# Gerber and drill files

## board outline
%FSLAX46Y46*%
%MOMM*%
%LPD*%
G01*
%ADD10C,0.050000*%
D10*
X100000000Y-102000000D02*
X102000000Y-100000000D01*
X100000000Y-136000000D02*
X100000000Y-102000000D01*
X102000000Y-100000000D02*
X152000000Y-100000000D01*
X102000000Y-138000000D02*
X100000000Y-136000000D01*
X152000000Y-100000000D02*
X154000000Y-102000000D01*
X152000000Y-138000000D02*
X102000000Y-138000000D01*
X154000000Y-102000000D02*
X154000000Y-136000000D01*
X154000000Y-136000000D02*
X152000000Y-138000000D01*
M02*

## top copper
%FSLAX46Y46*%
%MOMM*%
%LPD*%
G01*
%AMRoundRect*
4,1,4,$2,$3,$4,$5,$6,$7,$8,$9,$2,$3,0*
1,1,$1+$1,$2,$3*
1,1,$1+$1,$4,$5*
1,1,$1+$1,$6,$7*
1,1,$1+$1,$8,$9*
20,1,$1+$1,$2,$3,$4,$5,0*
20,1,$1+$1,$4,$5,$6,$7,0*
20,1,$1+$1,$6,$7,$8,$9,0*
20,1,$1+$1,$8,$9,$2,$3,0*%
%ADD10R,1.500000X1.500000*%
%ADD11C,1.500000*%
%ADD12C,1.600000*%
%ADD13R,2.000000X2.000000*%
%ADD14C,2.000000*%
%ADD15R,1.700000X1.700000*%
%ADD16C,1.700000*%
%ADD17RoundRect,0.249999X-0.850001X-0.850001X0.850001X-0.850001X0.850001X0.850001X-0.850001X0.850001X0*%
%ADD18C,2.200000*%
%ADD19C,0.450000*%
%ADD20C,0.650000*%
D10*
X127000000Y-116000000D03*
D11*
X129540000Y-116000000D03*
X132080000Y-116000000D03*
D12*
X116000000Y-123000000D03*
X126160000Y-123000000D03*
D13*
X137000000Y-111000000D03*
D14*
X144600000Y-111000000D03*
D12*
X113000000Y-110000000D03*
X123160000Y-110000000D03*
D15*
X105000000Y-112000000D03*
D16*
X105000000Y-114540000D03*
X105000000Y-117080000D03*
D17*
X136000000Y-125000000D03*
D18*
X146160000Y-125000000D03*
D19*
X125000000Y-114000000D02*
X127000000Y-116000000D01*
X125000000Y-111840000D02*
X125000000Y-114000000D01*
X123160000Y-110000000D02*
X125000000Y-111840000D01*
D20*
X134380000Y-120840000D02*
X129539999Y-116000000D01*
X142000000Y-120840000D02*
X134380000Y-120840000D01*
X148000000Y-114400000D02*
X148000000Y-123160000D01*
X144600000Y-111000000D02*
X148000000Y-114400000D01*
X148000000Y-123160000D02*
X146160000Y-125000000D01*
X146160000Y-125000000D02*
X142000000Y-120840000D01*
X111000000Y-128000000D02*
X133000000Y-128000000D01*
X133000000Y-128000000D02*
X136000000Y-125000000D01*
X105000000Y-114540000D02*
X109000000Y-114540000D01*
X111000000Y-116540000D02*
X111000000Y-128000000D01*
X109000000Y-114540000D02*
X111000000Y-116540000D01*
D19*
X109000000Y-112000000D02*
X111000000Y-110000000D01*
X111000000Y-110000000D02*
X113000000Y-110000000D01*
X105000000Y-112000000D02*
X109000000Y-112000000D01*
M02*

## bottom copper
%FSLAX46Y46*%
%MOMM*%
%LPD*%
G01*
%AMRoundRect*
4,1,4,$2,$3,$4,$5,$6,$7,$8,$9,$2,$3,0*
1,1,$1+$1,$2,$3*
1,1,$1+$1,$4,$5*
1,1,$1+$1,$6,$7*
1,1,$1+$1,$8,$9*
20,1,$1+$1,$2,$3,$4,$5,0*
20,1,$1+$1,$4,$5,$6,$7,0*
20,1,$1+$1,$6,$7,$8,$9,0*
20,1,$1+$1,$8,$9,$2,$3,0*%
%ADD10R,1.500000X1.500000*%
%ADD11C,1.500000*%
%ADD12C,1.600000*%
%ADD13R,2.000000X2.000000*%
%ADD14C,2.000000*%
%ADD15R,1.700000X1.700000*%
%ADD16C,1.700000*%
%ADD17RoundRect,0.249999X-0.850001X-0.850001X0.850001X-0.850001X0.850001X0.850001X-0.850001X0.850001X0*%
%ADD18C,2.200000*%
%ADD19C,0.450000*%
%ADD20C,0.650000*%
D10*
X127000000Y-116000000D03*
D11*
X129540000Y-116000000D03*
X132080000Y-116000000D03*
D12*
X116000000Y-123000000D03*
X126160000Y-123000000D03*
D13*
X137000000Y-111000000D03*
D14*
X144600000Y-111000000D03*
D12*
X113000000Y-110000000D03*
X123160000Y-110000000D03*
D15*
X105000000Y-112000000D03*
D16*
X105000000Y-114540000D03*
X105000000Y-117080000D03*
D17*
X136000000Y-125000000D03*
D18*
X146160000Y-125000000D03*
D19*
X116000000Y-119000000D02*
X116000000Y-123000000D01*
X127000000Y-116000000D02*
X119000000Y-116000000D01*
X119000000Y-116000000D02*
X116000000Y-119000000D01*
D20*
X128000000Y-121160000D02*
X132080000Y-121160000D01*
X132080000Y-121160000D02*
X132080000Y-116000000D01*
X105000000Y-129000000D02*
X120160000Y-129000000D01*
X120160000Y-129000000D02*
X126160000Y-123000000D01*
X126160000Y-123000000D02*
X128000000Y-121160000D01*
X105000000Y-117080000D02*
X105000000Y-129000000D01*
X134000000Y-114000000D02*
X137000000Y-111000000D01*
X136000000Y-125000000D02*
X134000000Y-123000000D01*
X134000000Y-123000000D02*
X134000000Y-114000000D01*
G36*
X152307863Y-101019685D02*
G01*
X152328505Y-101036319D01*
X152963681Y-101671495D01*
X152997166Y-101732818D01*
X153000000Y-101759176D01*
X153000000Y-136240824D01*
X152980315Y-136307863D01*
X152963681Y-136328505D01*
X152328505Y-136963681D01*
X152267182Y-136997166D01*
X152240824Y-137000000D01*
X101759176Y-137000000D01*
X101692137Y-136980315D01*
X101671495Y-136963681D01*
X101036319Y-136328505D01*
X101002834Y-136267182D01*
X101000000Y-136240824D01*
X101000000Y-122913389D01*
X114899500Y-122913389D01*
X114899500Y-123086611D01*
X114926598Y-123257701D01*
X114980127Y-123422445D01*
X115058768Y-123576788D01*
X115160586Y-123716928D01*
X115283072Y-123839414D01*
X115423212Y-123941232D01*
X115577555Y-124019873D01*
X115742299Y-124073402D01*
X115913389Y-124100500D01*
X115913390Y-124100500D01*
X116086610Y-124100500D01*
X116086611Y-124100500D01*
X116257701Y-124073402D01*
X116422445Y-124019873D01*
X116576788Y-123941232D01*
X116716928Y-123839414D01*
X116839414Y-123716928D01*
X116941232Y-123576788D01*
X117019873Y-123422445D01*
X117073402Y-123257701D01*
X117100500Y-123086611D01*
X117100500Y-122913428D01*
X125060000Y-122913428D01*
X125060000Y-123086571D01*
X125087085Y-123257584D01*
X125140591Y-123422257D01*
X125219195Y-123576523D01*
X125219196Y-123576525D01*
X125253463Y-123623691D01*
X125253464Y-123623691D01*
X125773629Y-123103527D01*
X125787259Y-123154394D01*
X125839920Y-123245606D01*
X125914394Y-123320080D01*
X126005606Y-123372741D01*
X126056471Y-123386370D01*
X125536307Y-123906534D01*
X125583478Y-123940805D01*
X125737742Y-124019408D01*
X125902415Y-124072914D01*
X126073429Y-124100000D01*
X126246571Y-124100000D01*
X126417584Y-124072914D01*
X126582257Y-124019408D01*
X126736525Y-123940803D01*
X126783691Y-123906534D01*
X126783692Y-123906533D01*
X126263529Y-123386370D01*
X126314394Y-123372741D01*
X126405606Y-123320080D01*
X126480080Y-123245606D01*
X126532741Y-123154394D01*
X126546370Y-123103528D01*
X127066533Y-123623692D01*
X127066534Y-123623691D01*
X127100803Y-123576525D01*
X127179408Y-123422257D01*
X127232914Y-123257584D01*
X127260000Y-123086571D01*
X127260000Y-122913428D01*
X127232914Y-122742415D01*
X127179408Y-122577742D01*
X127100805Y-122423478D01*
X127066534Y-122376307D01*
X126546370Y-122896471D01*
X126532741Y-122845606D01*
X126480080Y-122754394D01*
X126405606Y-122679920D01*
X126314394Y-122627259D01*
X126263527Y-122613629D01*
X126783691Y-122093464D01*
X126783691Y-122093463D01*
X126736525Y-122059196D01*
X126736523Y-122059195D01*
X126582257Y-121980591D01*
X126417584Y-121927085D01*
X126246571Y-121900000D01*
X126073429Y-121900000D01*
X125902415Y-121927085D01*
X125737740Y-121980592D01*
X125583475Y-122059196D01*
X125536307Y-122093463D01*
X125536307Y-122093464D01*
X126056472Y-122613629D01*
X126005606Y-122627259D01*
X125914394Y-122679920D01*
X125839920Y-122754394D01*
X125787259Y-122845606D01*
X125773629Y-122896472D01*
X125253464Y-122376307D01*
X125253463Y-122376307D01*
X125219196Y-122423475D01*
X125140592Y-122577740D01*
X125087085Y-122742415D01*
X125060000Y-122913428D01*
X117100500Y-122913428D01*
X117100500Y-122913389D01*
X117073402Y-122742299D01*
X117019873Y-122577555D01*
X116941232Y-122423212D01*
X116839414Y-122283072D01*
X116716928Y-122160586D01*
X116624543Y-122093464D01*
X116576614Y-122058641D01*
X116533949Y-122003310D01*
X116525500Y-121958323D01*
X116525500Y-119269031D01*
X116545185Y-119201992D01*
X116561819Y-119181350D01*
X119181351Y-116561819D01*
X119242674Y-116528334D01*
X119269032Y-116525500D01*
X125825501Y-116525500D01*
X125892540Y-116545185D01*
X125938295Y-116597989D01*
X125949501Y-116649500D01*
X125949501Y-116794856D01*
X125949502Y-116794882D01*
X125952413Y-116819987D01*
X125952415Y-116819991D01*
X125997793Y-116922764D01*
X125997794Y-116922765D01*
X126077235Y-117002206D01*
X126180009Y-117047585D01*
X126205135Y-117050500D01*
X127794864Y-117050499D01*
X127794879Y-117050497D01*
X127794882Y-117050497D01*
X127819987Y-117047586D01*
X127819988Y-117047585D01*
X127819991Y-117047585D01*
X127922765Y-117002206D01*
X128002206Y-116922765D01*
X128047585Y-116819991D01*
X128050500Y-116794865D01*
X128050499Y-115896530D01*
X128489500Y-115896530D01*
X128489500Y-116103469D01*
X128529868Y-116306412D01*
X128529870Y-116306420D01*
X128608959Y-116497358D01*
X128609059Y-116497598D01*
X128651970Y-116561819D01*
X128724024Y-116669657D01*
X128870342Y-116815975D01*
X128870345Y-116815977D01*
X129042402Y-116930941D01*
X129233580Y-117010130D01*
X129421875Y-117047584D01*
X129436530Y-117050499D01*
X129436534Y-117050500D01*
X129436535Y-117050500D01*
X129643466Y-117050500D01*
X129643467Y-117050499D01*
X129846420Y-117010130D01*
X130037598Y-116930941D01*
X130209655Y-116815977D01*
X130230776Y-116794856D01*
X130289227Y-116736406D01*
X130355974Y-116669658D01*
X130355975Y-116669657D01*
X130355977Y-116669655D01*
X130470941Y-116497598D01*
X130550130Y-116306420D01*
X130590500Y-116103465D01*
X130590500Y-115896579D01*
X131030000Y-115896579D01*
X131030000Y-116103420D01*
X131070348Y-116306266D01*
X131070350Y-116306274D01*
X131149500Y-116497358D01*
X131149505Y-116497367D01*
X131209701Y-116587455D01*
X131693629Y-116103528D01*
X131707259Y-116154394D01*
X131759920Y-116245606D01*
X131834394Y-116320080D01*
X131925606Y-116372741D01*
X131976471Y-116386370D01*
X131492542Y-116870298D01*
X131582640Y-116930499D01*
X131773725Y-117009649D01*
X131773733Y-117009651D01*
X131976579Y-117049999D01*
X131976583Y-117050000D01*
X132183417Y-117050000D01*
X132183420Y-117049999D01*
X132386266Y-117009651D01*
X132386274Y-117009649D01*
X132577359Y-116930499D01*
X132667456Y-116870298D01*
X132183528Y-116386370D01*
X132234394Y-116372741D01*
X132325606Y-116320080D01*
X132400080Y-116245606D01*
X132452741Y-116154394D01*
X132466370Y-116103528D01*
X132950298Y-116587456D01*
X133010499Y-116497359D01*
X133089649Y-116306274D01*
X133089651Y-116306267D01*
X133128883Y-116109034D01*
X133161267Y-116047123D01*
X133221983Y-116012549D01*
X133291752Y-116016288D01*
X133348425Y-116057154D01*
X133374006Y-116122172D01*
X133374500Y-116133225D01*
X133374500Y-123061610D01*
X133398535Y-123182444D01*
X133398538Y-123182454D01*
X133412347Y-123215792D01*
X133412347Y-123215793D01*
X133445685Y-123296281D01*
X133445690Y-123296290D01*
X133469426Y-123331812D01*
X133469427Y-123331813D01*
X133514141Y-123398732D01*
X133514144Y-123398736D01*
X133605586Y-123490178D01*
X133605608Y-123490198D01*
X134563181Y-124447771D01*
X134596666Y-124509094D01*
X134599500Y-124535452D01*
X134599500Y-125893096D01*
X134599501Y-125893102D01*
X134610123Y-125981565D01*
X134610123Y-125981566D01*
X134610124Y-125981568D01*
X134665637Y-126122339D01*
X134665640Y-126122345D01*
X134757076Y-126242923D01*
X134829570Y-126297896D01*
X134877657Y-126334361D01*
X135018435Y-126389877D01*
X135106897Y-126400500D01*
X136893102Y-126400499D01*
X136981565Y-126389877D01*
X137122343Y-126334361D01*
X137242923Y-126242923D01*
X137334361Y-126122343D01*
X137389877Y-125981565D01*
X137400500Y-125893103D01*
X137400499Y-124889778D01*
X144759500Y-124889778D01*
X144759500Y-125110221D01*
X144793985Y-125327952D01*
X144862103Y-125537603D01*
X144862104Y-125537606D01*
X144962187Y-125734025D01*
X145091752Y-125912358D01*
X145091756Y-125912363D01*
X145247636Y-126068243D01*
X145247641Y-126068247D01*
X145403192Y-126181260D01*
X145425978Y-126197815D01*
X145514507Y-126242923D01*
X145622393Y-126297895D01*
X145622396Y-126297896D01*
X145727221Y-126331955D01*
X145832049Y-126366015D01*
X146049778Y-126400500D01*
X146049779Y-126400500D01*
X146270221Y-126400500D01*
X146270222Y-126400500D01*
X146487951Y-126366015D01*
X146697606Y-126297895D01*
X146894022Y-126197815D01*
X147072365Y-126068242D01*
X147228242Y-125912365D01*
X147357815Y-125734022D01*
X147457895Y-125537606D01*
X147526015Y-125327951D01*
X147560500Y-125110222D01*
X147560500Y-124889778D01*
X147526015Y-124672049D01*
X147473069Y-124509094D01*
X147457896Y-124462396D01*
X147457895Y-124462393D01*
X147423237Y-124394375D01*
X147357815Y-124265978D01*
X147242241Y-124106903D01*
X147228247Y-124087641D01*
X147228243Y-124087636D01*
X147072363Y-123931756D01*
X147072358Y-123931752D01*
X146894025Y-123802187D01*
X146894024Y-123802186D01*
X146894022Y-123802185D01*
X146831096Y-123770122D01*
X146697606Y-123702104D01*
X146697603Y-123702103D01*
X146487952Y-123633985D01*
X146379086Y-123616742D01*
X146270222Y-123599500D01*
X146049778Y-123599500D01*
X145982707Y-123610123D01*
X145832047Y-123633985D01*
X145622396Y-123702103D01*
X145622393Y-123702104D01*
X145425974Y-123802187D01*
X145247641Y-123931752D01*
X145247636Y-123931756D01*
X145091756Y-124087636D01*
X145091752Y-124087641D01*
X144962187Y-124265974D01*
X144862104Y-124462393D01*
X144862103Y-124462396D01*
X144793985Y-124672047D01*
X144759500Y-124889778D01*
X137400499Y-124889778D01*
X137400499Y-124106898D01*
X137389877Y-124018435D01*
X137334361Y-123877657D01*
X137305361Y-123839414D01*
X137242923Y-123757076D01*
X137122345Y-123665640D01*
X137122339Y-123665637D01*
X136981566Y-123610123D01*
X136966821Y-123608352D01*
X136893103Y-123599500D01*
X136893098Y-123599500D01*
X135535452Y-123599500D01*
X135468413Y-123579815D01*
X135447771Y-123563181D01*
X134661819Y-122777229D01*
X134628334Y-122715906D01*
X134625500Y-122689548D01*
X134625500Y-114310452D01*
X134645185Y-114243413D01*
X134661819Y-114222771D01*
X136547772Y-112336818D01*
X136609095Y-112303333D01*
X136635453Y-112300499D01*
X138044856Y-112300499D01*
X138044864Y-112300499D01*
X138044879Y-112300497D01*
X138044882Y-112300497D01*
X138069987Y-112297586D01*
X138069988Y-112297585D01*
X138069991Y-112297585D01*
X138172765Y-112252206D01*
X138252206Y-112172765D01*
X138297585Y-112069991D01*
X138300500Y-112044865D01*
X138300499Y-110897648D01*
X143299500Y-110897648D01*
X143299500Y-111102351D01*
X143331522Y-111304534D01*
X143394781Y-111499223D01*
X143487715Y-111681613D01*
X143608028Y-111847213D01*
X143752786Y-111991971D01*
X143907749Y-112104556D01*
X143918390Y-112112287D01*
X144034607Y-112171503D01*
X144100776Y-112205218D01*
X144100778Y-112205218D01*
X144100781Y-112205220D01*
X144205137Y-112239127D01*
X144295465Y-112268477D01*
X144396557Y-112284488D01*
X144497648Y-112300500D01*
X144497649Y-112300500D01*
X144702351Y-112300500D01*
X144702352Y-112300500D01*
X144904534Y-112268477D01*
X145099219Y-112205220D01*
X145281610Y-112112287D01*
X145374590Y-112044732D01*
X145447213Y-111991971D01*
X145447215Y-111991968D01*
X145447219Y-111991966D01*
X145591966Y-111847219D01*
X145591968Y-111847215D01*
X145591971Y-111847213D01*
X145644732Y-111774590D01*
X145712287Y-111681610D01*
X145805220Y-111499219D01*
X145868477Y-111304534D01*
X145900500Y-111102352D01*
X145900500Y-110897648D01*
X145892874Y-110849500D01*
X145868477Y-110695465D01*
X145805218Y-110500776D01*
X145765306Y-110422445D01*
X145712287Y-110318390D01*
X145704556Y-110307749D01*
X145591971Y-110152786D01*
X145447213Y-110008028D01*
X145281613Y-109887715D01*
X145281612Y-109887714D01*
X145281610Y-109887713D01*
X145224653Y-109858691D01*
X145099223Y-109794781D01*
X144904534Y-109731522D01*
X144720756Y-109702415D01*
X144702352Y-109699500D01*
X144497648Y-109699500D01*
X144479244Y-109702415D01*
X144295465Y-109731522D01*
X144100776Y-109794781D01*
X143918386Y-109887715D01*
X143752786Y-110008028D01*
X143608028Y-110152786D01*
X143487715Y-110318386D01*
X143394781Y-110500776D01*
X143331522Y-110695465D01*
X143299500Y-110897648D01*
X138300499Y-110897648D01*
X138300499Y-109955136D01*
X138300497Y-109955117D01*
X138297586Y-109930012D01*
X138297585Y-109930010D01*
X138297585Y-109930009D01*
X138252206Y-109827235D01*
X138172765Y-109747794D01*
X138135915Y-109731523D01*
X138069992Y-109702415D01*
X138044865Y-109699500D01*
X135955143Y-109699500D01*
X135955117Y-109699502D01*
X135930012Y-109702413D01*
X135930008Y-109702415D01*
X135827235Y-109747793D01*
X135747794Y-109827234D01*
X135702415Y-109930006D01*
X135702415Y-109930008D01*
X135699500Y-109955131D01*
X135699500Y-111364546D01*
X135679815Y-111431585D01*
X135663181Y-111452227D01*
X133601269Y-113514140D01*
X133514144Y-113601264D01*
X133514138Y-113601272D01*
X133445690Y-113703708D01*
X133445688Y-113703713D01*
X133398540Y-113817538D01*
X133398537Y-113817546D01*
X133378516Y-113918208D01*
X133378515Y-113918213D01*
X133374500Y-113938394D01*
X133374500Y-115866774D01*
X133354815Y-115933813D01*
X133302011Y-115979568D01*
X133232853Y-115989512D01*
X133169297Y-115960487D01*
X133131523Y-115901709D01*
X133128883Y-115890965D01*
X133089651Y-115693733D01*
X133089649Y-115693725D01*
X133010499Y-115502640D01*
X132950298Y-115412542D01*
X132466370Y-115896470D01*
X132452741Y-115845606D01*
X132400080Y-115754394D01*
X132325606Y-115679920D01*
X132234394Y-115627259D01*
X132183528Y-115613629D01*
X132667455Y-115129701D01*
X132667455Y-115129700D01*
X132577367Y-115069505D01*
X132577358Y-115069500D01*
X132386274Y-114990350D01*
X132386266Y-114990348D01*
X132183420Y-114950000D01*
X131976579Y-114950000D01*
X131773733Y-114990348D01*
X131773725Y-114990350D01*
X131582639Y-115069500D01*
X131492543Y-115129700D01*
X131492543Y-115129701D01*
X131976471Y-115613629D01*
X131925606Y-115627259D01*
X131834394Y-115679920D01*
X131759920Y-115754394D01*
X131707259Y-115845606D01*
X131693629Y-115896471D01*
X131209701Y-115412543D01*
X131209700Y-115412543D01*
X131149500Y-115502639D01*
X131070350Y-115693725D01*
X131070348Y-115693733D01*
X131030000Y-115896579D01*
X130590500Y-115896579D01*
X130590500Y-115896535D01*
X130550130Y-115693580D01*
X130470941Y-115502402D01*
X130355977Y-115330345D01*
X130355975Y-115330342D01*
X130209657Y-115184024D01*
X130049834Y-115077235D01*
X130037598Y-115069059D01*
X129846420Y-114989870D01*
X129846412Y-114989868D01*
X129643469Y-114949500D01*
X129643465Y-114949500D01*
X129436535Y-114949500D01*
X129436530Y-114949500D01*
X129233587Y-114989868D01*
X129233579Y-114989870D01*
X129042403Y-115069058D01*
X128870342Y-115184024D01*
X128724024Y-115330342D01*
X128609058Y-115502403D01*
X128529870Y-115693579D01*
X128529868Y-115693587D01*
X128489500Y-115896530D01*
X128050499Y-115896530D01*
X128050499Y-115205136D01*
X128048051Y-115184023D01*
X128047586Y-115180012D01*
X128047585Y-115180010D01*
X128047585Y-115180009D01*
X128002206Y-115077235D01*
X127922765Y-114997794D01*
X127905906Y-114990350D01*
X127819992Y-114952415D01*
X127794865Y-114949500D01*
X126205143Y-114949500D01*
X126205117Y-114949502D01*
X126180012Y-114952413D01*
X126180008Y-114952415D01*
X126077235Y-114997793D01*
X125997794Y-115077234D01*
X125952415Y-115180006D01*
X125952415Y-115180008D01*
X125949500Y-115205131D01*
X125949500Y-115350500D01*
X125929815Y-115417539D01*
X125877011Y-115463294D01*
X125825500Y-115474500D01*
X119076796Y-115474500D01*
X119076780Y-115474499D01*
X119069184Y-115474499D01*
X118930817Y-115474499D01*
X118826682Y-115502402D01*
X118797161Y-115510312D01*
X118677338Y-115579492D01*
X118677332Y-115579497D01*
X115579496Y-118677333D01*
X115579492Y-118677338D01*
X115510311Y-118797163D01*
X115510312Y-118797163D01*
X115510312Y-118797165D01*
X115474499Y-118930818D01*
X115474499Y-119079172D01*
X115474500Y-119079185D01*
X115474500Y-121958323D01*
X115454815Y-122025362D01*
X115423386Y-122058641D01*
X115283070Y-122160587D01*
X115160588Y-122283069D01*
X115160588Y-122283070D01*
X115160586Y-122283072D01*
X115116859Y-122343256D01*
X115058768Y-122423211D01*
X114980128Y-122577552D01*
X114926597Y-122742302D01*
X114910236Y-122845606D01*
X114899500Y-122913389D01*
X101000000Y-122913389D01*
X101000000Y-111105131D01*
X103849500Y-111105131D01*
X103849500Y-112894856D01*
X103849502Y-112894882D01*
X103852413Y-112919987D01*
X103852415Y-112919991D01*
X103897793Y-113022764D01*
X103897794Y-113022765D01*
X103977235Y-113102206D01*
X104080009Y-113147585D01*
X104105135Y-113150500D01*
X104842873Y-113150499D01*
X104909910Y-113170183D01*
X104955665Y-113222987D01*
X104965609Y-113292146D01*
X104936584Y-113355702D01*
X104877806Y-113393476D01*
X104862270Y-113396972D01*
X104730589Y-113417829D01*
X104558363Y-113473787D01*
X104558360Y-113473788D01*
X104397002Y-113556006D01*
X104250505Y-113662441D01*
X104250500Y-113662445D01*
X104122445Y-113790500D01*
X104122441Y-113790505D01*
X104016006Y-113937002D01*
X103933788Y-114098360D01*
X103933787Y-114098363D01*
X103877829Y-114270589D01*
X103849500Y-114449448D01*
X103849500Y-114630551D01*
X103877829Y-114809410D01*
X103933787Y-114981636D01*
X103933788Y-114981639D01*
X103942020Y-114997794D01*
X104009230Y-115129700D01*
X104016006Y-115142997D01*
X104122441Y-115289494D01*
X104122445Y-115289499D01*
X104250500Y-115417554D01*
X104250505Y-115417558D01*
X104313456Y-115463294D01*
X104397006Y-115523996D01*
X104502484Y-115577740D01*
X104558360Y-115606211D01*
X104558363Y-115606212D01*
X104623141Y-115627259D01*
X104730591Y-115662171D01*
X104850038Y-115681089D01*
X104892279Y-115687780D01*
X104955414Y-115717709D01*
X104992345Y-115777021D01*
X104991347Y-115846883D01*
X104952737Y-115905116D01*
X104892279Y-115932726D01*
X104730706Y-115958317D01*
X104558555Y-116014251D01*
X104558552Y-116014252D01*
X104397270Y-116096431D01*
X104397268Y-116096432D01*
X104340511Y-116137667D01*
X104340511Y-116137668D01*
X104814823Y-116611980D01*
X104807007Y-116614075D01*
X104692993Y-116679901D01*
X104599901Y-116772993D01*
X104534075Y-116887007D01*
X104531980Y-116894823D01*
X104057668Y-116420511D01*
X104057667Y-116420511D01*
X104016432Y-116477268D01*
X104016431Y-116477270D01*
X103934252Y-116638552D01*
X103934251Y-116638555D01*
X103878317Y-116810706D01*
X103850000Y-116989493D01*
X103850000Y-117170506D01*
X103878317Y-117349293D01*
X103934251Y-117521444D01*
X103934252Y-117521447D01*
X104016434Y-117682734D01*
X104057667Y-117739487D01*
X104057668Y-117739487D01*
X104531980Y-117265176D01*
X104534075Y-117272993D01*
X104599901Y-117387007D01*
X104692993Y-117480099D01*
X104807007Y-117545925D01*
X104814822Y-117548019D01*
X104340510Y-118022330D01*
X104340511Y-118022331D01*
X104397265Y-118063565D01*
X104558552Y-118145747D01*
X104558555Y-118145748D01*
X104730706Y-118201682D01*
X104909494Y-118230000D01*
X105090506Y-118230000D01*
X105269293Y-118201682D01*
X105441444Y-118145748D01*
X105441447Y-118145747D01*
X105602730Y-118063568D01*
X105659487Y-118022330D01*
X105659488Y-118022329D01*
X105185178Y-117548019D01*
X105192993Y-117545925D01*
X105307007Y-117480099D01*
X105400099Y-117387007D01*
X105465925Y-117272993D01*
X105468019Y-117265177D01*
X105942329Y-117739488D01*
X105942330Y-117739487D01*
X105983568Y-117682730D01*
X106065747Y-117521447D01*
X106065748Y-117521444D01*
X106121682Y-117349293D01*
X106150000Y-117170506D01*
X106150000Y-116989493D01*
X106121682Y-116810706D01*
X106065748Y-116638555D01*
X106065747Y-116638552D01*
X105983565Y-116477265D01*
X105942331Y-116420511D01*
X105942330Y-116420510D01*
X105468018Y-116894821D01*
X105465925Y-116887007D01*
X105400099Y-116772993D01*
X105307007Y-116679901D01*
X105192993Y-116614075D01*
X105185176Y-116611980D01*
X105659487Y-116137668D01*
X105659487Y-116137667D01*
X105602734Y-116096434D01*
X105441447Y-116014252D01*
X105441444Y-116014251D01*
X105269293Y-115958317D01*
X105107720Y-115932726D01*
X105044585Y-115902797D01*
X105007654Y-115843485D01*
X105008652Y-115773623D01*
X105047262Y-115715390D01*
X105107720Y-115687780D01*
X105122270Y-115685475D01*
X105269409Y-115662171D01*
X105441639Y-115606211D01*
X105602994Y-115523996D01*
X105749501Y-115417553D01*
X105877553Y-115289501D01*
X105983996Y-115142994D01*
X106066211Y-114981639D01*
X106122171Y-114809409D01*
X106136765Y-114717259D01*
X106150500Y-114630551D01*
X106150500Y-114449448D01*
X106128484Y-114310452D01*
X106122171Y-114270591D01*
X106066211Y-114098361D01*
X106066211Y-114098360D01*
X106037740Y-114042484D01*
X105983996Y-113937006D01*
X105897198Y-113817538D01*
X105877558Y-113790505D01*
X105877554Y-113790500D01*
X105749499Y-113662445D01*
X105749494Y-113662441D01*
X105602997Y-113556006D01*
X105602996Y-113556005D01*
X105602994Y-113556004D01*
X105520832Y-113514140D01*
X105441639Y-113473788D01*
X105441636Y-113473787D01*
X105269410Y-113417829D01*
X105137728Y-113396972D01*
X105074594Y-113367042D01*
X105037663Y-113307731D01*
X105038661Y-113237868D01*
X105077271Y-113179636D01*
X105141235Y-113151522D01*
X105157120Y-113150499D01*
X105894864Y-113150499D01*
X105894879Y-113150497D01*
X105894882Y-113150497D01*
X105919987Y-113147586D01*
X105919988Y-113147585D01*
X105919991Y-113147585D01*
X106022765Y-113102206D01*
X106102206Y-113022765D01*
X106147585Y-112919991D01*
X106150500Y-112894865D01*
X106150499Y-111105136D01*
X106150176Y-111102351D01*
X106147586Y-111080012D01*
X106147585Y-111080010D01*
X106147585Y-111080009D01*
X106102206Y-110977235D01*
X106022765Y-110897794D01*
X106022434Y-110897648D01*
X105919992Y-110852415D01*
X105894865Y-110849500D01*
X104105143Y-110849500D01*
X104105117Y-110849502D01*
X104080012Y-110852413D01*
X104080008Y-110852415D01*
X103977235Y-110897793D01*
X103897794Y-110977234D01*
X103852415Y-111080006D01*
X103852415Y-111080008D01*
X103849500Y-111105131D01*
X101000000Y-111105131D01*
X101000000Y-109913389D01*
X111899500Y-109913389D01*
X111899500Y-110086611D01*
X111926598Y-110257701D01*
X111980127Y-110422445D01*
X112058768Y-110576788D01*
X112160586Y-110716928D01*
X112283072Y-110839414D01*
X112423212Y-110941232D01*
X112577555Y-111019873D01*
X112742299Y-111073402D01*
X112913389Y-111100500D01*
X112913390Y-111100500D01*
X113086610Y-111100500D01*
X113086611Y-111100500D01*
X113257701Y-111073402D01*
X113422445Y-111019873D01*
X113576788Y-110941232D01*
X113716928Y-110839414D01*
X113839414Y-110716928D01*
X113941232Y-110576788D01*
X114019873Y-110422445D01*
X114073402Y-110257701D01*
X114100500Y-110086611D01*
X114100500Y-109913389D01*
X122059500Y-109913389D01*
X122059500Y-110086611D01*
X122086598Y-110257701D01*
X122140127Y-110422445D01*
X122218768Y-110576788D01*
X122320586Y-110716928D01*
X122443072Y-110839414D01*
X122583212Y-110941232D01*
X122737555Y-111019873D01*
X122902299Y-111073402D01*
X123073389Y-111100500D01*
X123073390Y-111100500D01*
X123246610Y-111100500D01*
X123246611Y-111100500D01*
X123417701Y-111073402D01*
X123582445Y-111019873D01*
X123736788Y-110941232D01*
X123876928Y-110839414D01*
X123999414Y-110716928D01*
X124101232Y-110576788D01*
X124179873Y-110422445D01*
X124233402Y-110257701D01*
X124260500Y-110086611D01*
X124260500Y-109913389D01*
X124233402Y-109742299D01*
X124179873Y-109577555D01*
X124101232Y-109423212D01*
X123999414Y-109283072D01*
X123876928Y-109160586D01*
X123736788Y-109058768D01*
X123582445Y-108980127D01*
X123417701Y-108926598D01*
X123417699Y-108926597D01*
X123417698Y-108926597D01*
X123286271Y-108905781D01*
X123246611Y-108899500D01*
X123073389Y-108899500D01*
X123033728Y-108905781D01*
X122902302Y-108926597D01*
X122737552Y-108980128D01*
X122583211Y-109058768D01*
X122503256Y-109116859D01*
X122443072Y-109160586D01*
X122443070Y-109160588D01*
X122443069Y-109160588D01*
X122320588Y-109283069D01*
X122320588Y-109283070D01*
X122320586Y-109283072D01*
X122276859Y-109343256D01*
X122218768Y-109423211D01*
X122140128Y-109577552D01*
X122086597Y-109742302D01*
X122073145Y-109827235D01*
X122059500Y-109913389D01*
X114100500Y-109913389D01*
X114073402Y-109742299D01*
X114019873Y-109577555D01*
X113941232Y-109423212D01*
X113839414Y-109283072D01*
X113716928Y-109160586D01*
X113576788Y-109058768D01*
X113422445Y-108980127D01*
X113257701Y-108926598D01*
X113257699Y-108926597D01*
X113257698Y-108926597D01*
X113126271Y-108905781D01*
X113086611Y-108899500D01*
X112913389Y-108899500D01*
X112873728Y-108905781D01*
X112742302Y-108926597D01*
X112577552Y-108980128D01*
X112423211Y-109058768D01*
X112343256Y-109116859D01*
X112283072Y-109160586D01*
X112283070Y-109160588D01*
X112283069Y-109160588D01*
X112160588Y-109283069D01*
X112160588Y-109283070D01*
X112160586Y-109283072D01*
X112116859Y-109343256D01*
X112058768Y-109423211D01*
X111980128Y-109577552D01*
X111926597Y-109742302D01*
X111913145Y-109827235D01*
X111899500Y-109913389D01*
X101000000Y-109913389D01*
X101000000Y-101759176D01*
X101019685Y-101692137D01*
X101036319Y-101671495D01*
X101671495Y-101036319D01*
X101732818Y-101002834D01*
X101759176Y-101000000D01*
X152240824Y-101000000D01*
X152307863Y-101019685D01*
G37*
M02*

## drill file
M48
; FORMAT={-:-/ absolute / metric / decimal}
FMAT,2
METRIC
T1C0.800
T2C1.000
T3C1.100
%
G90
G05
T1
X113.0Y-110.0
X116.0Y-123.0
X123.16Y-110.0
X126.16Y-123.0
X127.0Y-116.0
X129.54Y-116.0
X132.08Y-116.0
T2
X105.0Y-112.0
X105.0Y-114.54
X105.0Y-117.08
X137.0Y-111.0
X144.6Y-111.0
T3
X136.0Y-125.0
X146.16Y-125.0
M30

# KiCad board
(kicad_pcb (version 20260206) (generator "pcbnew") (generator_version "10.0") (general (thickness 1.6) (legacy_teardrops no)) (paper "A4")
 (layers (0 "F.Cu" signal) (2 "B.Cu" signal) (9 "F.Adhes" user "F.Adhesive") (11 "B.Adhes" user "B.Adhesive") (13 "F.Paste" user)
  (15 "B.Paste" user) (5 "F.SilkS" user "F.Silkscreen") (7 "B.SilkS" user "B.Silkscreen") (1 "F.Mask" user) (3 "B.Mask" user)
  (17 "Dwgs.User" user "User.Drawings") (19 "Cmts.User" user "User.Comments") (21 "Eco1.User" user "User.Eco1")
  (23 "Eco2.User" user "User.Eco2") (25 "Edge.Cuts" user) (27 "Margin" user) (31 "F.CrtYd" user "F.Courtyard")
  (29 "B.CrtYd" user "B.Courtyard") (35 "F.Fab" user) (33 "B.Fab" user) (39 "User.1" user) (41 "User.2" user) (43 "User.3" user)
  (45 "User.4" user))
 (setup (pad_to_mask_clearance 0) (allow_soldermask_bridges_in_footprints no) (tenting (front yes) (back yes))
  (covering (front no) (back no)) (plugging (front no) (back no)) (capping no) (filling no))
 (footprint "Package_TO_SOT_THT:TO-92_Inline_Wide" (layer "F.Cu") (at 127 116)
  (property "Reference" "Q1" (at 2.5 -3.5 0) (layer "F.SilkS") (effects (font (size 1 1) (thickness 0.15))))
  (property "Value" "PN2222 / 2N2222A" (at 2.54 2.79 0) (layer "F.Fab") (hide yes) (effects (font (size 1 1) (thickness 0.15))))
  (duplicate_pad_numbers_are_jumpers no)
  (pad "1" thru_hole rect (at 0 0) (size 1.5 1.5) (drill 0.8) (layers "*.Cu" "*.Mask") (remove_unused_layers no) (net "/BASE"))
  (pad "2" thru_hole circle (at 2.54 0) (size 1.5 1.5) (drill 0.8) (layers "*.Cu" "*.Mask") (remove_unused_layers no) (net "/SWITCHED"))
  (pad "3" thru_hole circle (at 5.08 0) (size 1.5 1.5) (drill 0.8) (layers "*.Cu" "*.Mask") (remove_unused_layers no) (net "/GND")))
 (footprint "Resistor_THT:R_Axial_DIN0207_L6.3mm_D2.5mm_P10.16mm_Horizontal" (layer "F.Cu") (at 116 123)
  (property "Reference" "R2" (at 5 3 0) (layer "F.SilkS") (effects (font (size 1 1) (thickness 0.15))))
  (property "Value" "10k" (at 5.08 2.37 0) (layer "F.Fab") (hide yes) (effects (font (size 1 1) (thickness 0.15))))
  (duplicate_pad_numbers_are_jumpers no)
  (pad "1" thru_hole circle (at 0 0) (size 1.6 1.6) (drill 0.8) (layers "*.Cu" "*.Mask") (remove_unused_layers no) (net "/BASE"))
  (pad "2" thru_hole circle (at 10.16 0) (size 1.6 1.6) (drill 0.8) (layers "*.Cu" "*.Mask") (remove_unused_layers no) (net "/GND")))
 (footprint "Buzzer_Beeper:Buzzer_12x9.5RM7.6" (layer "F.Cu") (at 137 111)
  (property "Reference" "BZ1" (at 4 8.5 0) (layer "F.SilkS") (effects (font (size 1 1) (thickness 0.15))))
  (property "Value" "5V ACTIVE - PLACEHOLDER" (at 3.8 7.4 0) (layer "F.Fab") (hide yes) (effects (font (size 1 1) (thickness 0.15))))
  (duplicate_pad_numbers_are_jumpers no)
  (pad "1" thru_hole rect (at 0 0) (size 2 2) (drill 1) (layers "*.Cu" "*.Mask") (remove_unused_layers no) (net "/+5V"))
  (pad "2" thru_hole circle (at 7.6 0) (size 2 2) (drill 1) (layers "*.Cu" "*.Mask") (remove_unused_layers no) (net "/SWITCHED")))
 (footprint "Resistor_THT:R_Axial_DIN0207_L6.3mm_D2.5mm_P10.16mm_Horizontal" (layer "F.Cu") (at 113 110)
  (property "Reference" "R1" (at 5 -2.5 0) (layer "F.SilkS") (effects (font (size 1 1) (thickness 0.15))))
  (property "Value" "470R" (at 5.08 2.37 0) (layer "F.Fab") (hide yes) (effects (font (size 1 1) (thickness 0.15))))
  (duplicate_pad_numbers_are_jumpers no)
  (pad "1" thru_hole circle (at 0 0) (size 1.6 1.6) (drill 0.8) (layers "*.Cu" "*.Mask") (remove_unused_layers no) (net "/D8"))
  (pad "2" thru_hole circle (at 10.16 0) (size 1.6 1.6) (drill 0.8) (layers "*.Cu" "*.Mask") (remove_unused_layers no) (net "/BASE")))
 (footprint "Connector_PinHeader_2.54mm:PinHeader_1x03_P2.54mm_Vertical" (layer "F.Cu") (at 105 112)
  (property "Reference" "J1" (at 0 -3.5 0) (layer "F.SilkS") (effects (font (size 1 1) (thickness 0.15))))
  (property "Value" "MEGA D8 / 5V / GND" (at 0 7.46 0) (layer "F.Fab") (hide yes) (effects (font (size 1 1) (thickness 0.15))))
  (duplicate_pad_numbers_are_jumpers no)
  (pad "1" thru_hole rect (at 0 0) (size 1.7 1.7) (drill 1) (layers "*.Cu" "*.Mask") (remove_unused_layers no) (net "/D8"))
  (pad "2" thru_hole circle (at 0 2.54) (size 1.7 1.7) (drill 1) (layers "*.Cu" "*.Mask") (remove_unused_layers no) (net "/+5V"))
  (pad "3" thru_hole circle (at 0 5.08) (size 1.7 1.7) (drill 1) (layers "*.Cu" "*.Mask") (remove_unused_layers no) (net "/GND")))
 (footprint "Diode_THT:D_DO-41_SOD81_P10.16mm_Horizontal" (layer "F.Cu") (at 136 125)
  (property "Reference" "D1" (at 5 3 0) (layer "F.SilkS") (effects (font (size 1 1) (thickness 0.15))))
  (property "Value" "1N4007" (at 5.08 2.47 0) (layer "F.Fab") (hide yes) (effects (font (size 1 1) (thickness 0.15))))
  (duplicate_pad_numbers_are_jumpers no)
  (pad "1" thru_hole roundrect (at 0 0) (size 2.2 2.2) (drill 1.1) (layers "*.Cu" "*.Mask") (remove_unused_layers no)
   (roundrect_rratio 0.113636) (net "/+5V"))
  (pad "2" thru_hole circle (at 10.16 0) (size 2.2 2.2) (drill 1.1) (layers "*.Cu" "*.Mask") (remove_unused_layers no) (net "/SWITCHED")))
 (gr_line (start 100 102) (end 102 100) (stroke (width 0.05) (type default)) (layer "Edge.Cuts"))
 (gr_line (start 100 136) (end 100 102) (stroke (width 0.05) (type default)) (layer "Edge.Cuts"))
 (gr_line (start 102 100) (end 152 100) (stroke (width 0.05) (type default)) (layer "Edge.Cuts"))
 (gr_line (start 102 138) (end 100 136) (stroke (width 0.05) (type default)) (layer "Edge.Cuts"))
 (gr_line (start 152 100) (end 154 102) (stroke (width 0.05) (type default)) (layer "Edge.Cuts"))
 (gr_line (start 152 138) (end 102 138) (stroke (width 0.05) (type default)) (layer "Edge.Cuts"))
 (gr_line (start 154 102) (end 154 136) (stroke (width 0.05) (type default)) (layer "Edge.Cuts"))
 (gr_line (start 154 136) (end 152 138) (stroke (width 0.05) (type default)) (layer "Edge.Cuts"))
 (segment (start 125 114) (end 127 116) (width 0.45) (layer "F.Cu") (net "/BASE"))
 (segment (start 125 111.84) (end 125 114) (width 0.45) (layer "F.Cu") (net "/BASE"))
 (segment (start 123.16 110) (end 125 111.84) (width 0.45) (layer "F.Cu") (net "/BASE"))
 (segment (start 116 119) (end 116 123) (width 0.45) (layer "B.Cu") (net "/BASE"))
 (segment (start 127 116) (end 119 116) (width 0.45) (layer "B.Cu") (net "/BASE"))
 (segment (start 119 116) (end 116 119) (width 0.45) (layer "B.Cu") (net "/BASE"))
 (segment (start 134.38 120.84) (end 129.539999 116) (width 0.65) (layer "F.Cu") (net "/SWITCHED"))
 (segment (start 142 120.84) (end 134.38 120.84) (width 0.65) (layer "F.Cu") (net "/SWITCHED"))
 (segment (start 148 114.4) (end 148 123.16) (width 0.65) (layer "F.Cu") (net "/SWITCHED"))
 (segment (start 144.6 111) (end 148 114.4) (width 0.65) (layer "F.Cu") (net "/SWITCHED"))
 (segment (start 148 123.16) (end 146.16 125) (width 0.65) (layer "F.Cu") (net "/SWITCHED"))
 (segment (start 146.16 125) (end 142 120.84) (width 0.65) (layer "F.Cu") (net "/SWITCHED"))
 (segment (start 128 121.16) (end 132.08 121.16) (width 0.65) (layer "B.Cu") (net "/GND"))
 (segment (start 132.08 121.16) (end 132.08 116) (width 0.65) (layer "B.Cu") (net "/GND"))
 (segment (start 105 129) (end 120.16 129) (width 0.65) (layer "B.Cu") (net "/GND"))
 (segment (start 120.16 129) (end 126.16 123) (width 0.65) (layer "B.Cu") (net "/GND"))
 (segment (start 126.16 123) (end 128 121.16) (width 0.65) (layer "B.Cu") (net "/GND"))
 (segment (start 105 117.08) (end 105 129) (width 0.65) (layer "B.Cu") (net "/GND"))
 (segment (start 111 128) (end 133 128) (width 0.65) (layer "F.Cu") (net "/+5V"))
 (segment (start 133 128) (end 136 125) (width 0.65) (layer "F.Cu") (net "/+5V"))
 (segment (start 105 114.54) (end 109 114.54) (width 0.65) (layer "F.Cu") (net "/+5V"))
 (segment (start 111 116.54) (end 111 128) (width 0.65) (layer "F.Cu") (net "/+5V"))
 (segment (start 109 114.54) (end 111 116.54) (width 0.65) (layer "F.Cu") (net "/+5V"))
 (segment (start 134 114) (end 137 111) (width 0.65) (layer "B.Cu") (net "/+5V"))
 (segment (start 136 125) (end 134 123) (width 0.65) (layer "B.Cu") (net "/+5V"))
 (segment (start 134 123) (end 134 114) (width 0.65) (layer "B.Cu") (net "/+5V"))
 (segment (start 109 112) (end 111 110) (width 0.45) (layer "F.Cu") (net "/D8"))
 (segment (start 111 110) (end 113 110) (width 0.45) (layer "F.Cu") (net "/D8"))
 (segment (start 105 112) (end 109 112) (width 0.45) (layer "F.Cu") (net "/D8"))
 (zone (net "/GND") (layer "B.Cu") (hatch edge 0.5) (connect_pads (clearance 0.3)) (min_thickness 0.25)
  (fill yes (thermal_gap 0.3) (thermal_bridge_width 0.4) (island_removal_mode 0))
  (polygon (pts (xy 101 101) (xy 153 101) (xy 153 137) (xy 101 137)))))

